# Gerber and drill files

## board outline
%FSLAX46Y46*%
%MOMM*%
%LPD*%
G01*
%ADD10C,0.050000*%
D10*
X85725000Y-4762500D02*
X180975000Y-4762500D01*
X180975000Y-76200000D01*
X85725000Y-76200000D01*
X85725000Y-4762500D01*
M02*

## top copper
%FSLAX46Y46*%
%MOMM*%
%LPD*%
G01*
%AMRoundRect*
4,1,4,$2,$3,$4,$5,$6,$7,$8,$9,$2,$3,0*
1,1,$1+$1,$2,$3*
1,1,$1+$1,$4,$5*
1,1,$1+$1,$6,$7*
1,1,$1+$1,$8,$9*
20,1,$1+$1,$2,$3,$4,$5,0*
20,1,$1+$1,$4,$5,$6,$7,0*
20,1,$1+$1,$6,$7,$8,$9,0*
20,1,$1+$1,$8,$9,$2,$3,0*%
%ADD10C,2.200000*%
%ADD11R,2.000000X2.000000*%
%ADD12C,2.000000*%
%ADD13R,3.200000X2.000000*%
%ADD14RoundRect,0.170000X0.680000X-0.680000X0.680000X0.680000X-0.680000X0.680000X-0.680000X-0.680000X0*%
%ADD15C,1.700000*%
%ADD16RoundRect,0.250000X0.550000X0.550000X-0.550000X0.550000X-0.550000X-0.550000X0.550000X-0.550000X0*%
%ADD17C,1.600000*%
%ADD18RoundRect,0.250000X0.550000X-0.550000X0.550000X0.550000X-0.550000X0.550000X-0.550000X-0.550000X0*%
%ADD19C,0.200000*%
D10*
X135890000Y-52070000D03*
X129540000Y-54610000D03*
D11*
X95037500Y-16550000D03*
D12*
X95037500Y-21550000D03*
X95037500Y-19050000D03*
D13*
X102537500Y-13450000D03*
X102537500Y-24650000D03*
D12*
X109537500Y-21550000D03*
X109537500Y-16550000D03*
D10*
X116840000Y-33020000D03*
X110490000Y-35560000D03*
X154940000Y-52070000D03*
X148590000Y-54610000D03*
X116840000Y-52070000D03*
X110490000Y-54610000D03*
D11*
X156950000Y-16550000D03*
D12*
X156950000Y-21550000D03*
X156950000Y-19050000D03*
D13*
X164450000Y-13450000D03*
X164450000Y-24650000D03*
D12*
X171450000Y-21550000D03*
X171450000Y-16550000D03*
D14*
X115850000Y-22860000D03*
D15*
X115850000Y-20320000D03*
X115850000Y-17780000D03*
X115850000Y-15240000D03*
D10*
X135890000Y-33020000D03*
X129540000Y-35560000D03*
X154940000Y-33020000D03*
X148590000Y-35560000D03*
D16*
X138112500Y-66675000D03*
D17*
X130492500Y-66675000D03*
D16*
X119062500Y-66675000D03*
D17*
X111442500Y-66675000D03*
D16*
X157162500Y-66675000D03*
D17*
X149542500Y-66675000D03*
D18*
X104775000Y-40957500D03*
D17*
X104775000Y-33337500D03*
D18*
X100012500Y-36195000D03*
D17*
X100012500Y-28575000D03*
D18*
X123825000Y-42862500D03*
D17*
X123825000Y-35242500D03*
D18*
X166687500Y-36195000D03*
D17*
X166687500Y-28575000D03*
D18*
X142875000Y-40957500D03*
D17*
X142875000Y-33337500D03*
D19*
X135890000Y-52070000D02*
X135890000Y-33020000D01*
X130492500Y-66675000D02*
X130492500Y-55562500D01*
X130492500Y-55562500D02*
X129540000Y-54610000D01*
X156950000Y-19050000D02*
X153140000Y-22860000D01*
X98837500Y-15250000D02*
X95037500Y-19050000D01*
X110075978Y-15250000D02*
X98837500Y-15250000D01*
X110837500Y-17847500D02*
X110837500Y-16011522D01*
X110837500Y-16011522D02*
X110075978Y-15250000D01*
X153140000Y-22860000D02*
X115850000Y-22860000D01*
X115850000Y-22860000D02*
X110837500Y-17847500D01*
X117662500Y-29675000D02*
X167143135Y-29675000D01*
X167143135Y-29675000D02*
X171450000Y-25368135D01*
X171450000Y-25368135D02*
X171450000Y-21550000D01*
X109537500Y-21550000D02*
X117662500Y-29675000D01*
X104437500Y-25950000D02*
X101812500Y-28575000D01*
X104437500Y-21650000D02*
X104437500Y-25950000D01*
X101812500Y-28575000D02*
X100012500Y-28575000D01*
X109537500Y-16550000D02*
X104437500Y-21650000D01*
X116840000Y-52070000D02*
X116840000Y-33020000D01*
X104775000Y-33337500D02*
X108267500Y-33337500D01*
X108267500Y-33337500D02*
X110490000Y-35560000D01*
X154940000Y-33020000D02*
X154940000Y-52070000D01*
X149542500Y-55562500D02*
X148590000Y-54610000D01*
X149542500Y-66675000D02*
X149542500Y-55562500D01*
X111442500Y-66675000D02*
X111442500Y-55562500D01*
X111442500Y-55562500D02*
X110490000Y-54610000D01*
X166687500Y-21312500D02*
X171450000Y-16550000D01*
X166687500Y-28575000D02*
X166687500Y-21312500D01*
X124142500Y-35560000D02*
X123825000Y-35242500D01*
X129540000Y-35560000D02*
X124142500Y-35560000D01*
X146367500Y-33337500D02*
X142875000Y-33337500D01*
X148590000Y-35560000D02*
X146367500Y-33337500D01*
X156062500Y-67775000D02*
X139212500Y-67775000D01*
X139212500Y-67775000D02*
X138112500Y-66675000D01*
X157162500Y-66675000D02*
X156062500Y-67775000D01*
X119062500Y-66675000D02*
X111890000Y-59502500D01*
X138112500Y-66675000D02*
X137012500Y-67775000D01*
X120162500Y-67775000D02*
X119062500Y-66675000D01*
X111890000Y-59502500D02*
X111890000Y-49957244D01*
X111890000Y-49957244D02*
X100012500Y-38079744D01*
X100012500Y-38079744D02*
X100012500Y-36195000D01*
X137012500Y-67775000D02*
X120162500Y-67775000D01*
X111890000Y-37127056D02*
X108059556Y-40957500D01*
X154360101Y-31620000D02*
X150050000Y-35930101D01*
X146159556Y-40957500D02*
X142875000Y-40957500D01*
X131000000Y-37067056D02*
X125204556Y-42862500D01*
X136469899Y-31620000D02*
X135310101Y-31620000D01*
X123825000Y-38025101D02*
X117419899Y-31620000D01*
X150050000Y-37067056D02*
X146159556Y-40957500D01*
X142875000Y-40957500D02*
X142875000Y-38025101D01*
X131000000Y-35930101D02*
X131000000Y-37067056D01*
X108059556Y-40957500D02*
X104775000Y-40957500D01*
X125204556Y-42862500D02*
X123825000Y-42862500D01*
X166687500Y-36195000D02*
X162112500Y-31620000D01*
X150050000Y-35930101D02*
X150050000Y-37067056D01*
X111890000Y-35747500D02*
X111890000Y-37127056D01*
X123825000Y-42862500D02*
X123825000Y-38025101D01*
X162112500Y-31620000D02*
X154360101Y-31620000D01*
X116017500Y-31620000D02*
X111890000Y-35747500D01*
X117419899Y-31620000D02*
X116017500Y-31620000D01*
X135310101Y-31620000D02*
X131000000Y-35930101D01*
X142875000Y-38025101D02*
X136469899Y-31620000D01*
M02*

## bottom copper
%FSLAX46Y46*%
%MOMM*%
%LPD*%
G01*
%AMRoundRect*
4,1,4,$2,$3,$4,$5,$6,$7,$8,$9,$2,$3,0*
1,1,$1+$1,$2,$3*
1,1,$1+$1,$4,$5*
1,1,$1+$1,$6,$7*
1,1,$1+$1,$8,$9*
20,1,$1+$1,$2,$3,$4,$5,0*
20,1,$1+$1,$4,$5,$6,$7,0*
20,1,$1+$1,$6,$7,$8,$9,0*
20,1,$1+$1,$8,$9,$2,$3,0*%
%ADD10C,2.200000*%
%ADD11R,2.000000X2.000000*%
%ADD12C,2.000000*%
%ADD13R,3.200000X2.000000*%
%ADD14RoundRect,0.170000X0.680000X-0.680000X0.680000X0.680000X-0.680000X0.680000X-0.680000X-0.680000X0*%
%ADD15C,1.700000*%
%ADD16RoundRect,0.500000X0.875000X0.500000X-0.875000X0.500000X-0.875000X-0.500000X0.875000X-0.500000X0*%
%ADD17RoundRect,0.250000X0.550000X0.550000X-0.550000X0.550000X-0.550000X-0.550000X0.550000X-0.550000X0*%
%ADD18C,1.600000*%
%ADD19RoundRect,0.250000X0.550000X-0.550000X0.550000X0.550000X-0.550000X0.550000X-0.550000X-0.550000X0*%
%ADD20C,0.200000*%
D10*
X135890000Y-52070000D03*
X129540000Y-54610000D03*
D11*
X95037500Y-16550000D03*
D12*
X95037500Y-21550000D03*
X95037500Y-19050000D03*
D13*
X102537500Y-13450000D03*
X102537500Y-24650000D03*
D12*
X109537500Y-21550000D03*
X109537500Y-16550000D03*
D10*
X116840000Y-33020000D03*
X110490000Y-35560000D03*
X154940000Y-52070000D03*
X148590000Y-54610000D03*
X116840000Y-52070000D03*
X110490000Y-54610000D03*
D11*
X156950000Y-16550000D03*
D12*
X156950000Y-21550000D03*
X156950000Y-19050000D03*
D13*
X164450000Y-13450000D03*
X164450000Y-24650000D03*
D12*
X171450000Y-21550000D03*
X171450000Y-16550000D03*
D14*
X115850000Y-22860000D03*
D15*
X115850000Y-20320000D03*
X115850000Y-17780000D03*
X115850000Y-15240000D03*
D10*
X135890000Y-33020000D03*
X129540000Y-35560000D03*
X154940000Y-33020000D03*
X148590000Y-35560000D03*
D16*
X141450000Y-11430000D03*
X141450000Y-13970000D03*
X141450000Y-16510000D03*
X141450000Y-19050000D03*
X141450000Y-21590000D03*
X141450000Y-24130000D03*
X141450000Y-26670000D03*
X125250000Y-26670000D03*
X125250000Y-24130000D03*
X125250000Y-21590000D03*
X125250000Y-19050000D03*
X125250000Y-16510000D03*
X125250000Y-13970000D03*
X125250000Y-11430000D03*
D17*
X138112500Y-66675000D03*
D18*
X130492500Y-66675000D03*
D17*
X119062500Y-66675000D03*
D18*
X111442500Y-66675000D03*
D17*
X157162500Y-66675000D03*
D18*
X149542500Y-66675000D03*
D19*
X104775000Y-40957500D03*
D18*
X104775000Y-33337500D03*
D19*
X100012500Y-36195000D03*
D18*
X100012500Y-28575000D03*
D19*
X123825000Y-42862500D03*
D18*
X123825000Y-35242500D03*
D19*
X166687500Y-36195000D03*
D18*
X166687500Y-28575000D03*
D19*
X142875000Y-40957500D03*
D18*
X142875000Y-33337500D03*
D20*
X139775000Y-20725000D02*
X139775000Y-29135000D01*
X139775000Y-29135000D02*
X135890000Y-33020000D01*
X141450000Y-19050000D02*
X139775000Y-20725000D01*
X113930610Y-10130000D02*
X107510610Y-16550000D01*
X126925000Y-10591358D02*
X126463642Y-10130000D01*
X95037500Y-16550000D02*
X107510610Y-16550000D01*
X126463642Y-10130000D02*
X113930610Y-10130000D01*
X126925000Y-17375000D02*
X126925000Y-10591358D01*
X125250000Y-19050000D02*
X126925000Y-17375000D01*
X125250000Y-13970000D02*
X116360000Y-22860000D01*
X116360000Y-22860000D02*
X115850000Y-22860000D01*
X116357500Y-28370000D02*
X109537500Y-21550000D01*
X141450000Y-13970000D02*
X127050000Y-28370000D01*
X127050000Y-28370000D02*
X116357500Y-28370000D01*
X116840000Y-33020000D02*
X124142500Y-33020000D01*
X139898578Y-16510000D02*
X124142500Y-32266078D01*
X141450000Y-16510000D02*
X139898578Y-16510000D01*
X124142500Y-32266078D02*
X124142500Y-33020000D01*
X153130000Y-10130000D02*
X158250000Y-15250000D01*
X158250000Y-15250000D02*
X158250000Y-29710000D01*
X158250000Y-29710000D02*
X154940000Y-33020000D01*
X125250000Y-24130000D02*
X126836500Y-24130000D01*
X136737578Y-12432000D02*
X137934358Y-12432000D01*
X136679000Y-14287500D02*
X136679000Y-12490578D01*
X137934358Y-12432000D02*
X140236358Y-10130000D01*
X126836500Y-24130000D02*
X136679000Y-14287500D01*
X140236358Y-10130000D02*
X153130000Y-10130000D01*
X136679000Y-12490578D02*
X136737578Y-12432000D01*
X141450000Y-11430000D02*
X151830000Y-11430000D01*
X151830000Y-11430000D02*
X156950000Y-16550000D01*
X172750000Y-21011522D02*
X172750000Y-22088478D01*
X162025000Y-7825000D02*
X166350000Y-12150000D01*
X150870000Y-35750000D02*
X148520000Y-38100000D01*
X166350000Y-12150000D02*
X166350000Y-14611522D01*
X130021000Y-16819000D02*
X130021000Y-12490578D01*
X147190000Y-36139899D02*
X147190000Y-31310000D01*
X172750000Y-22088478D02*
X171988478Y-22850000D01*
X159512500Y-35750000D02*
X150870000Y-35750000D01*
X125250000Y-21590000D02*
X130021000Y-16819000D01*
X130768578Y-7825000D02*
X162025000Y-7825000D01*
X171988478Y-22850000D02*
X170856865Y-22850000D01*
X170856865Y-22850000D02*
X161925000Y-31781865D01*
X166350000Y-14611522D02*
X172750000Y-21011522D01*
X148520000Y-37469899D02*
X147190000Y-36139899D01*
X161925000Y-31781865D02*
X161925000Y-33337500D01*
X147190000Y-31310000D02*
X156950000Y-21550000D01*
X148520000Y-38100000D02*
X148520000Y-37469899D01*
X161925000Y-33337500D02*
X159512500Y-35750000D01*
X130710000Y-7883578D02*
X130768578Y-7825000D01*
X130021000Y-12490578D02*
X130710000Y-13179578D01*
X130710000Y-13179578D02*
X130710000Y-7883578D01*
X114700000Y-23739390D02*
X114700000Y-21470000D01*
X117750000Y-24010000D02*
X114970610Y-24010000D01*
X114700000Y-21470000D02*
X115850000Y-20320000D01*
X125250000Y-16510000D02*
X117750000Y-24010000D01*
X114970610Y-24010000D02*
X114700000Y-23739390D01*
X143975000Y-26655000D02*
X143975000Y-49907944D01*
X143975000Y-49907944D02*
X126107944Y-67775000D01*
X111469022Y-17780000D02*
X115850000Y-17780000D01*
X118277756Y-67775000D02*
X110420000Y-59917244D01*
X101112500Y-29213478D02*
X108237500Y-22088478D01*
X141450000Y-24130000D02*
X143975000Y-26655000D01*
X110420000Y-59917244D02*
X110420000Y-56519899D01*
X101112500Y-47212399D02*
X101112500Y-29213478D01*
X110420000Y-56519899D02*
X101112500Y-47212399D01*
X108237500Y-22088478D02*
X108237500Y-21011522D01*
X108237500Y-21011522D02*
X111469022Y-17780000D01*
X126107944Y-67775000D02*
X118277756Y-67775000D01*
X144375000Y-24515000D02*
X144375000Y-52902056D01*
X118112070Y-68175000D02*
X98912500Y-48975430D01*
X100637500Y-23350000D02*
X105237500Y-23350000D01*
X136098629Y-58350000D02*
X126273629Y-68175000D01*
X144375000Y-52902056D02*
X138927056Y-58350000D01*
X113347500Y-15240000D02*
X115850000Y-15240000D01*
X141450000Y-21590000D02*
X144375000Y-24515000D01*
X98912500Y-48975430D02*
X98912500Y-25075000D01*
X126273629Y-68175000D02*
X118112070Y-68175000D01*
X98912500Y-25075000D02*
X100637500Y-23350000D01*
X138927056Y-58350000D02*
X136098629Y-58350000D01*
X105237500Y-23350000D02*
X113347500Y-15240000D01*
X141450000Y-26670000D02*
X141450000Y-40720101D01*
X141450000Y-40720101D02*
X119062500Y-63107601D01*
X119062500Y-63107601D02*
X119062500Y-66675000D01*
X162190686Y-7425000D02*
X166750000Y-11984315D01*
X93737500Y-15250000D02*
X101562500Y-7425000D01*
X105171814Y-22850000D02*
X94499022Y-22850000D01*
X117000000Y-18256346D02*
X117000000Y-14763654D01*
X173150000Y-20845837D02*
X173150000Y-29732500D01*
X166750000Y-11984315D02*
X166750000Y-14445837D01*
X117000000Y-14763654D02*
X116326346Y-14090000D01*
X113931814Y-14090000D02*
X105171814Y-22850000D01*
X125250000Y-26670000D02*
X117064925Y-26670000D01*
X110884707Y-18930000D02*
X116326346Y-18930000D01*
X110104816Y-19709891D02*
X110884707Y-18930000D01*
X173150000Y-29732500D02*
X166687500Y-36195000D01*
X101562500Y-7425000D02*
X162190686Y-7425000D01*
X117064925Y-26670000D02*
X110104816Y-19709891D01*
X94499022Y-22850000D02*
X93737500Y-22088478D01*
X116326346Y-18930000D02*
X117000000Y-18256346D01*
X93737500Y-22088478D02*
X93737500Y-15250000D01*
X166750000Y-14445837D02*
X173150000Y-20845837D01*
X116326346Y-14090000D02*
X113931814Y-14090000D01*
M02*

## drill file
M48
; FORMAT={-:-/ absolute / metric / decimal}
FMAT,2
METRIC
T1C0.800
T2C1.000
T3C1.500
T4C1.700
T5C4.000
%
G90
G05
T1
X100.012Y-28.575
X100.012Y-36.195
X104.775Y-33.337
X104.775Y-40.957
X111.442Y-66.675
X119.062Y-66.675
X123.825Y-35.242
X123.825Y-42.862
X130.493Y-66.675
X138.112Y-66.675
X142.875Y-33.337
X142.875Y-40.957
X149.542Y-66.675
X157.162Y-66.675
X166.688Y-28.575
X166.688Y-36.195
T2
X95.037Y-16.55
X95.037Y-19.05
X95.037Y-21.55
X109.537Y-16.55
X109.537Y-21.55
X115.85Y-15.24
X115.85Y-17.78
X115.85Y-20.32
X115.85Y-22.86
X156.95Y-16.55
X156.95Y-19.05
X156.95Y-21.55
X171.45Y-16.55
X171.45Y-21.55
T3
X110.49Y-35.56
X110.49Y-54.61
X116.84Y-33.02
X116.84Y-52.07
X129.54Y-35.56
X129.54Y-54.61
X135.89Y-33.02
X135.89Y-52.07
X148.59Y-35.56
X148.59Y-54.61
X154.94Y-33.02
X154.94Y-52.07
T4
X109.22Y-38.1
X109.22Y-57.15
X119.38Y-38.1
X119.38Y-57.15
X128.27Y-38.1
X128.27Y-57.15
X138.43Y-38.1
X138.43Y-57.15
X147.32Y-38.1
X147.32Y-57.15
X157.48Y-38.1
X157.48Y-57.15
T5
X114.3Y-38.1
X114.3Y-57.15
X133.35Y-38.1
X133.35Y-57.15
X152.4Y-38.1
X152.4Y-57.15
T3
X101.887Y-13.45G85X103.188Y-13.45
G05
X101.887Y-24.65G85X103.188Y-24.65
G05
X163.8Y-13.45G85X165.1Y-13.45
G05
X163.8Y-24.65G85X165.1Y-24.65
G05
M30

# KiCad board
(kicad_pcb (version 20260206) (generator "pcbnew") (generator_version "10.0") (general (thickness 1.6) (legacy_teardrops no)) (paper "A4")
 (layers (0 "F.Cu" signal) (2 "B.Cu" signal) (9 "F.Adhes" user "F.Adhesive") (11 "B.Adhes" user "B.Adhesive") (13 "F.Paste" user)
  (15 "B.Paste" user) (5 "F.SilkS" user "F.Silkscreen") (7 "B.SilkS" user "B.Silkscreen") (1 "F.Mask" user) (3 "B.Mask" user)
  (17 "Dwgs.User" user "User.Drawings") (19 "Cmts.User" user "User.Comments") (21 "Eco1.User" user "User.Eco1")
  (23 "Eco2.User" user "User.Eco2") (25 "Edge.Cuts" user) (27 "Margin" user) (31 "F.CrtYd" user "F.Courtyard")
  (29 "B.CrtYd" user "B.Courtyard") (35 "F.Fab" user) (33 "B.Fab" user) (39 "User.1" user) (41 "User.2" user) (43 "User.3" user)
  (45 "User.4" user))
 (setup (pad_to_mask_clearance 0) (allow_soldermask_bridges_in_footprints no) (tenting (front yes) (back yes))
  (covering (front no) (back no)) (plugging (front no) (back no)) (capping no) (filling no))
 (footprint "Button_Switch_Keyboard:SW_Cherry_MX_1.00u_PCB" (layer "F.Cu") (at 135.89 52.07)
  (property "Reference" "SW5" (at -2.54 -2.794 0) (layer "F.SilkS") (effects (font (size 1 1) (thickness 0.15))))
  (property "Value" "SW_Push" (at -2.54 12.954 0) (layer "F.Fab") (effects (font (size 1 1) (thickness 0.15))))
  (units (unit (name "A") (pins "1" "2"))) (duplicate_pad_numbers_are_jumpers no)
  (pad "" np_thru_hole circle (at -7.62 5.08) (size 1.7 1.7) (drill 1.7) (layers "*.Cu" "*.Mask"))
  (pad "" np_thru_hole circle (at -2.54 5.08) (size 4 4) (drill 4) (layers "*.Cu" "*.Mask"))
  (pad "" np_thru_hole circle (at 2.54 5.08) (size 1.7 1.7) (drill 1.7) (layers "*.Cu" "*.Mask"))
  (pad "1" thru_hole circle (at 0 0) (size 2.2 2.2) (drill 1.5) (layers "*.Cu" "*.Mask") (remove_unused_layers no) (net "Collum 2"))
  (pad "2" thru_hole circle (at -6.35 2.54) (size 2.2 2.2) (drill 1.5) (layers "*.Cu" "*.Mask") (remove_unused_layers no) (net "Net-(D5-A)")))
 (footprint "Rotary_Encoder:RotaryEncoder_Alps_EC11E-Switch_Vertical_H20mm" (layer "F.Cu") (at 95.0375 16.55)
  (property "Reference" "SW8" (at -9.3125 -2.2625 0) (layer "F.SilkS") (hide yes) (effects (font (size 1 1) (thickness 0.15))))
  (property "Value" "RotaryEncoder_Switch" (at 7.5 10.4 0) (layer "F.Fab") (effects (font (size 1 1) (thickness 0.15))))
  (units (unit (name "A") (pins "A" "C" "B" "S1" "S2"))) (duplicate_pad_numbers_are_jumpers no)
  (pad "A" thru_hole rect (at 0 0) (size 2 2) (drill 1) (layers "*.Cu" "*.Mask") (remove_unused_layers no) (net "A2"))
  (pad "B" thru_hole circle (at 0 5) (size 2 2) (drill 1) (layers "*.Cu" "*.Mask") (remove_unused_layers no) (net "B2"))
  (pad "C" thru_hole circle (at 0 2.5) (size 2 2) (drill 1) (layers "*.Cu" "*.Mask") (remove_unused_layers no) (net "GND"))
  (pad "MP" thru_hole rect (at 7.5 -3.1) (size 3.2 2) (drill oval 2.8 1.5) (layers "*.Cu" "*.Mask") (remove_unused_layers no))
  (pad "MP" thru_hole rect (at 7.5 8.1) (size 3.2 2) (drill oval 2.8 1.5) (layers "*.Cu" "*.Mask") (remove_unused_layers no))
  (pad "S1" thru_hole circle (at 14.5 5) (size 2 2) (drill 1) (layers "*.Cu" "*.Mask") (remove_unused_layers no) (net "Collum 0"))
  (pad "S2" thru_hole circle (at 14.5 0) (size 2 2) (drill 1) (layers "*.Cu" "*.Mask") (remove_unused_layers no) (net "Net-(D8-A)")))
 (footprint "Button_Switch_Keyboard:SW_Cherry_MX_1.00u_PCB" (layer "F.Cu") (at 116.84 33.02)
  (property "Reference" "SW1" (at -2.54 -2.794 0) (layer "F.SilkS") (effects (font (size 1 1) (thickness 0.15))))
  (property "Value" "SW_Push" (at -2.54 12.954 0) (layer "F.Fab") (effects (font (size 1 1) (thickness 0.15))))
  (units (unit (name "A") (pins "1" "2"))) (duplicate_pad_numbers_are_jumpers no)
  (pad "" np_thru_hole circle (at -7.62 5.08) (size 1.7 1.7) (drill 1.7) (layers "*.Cu" "*.Mask"))
  (pad "" np_thru_hole circle (at -2.54 5.08) (size 4 4) (drill 4) (layers "*.Cu" "*.Mask"))
  (pad "" np_thru_hole circle (at 2.54 5.08) (size 1.7 1.7) (drill 1.7) (layers "*.Cu" "*.Mask"))
  (pad "1" thru_hole circle (at 0 0) (size 2.2 2.2) (drill 1.5) (layers "*.Cu" "*.Mask") (remove_unused_layers no) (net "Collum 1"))
  (pad "2" thru_hole circle (at -6.35 2.54) (size 2.2 2.2) (drill 1.5) (layers "*.Cu" "*.Mask") (remove_unused_layers no) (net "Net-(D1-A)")))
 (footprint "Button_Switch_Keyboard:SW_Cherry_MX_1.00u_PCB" (layer "F.Cu") (at 154.94 52.07)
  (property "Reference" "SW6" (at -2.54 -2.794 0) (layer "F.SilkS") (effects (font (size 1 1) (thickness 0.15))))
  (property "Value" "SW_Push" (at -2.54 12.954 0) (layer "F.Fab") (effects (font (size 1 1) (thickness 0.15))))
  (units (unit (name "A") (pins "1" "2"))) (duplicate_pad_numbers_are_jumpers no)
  (pad "" np_thru_hole circle (at -7.62 5.08) (size 1.7 1.7) (drill 1.7) (layers "*.Cu" "*.Mask"))
  (pad "" np_thru_hole circle (at -2.54 5.08) (size 4 4) (drill 4) (layers "*.Cu" "*.Mask"))
  (pad "" np_thru_hole circle (at 2.54 5.08) (size 1.7 1.7) (drill 1.7) (layers "*.Cu" "*.Mask"))
  (pad "1" thru_hole circle (at 0 0) (size 2.2 2.2) (drill 1.5) (layers "*.Cu" "*.Mask") (remove_unused_layers no) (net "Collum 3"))
  (pad "2" thru_hole circle (at -6.35 2.54) (size 2.2 2.2) (drill 1.5) (layers "*.Cu" "*.Mask") (remove_unused_layers no) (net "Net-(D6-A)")))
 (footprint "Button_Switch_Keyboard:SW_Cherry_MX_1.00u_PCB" (layer "F.Cu") (at 116.84 52.07)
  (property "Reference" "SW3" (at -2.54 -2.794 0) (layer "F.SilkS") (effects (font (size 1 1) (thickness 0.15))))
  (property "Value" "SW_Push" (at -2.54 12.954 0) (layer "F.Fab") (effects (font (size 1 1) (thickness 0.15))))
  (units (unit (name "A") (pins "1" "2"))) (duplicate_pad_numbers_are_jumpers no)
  (pad "" np_thru_hole circle (at -7.62 5.08) (size 1.7 1.7) (drill 1.7) (layers "*.Cu" "*.Mask"))
  (pad "" np_thru_hole circle (at -2.54 5.08) (size 4 4) (drill 4) (layers "*.Cu" "*.Mask"))
  (pad "" np_thru_hole circle (at 2.54 5.08) (size 1.7 1.7) (drill 1.7) (layers "*.Cu" "*.Mask"))
  (pad "1" thru_hole circle (at 0 0) (size 2.2 2.2) (drill 1.5) (layers "*.Cu" "*.Mask") (remove_unused_layers no) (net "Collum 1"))
  (pad "2" thru_hole circle (at -6.35 2.54) (size 2.2 2.2) (drill 1.5) (layers "*.Cu" "*.Mask") (remove_unused_layers no) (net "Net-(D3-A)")))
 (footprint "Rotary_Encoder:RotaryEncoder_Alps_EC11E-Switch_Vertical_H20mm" (layer "F.Cu") (at 156.95 16.55)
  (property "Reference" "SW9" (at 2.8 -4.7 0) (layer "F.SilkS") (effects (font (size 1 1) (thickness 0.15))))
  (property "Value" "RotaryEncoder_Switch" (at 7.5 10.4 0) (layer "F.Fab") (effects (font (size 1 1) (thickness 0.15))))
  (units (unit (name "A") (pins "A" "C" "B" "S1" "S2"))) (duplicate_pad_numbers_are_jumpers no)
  (pad "A" thru_hole rect (at 0 0) (size 2 2) (drill 1) (layers "*.Cu" "*.Mask") (remove_unused_layers no) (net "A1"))
  (pad "B" thru_hole circle (at 0 5) (size 2 2) (drill 1) (layers "*.Cu" "*.Mask") (remove_unused_layers no) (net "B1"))
  (pad "C" thru_hole circle (at 0 2.5) (size 2 2) (drill 1) (layers "*.Cu" "*.Mask") (remove_unused_layers no) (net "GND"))
  (pad "MP" thru_hole rect (at 7.5 -3.1) (size 3.2 2) (drill oval 2.8 1.5) (layers "*.Cu" "*.Mask") (remove_unused_layers no))
  (pad "MP" thru_hole rect (at 7.5 8.1) (size 3.2 2) (drill oval 2.8 1.5) (layers "*.Cu" "*.Mask") (remove_unused_layers no))
  (pad "S1" thru_hole circle (at 14.5 5) (size 2 2) (drill 1) (layers "*.Cu" "*.Mask") (remove_unused_layers no) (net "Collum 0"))
  (pad "S2" thru_hole circle (at 14.5 0) (size 2 2) (drill 1) (layers "*.Cu" "*.Mask") (remove_unused_layers no) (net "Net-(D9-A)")))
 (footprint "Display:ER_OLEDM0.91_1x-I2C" (layer "F.Cu") (at 115.85 22.86 90)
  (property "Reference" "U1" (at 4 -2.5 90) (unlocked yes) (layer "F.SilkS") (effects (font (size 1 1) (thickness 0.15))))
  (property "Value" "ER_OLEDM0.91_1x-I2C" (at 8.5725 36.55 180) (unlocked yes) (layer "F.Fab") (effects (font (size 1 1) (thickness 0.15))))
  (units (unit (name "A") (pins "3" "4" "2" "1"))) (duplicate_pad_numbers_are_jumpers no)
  (pad "1" thru_hole roundrect (at 0 0 90) (size 1.7 1.7) (drill 1) (layers "*.Cu" "*.Mask") (remove_unused_layers no)
   (roundrect_rratio 0.1) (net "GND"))
  (pad "2" thru_hole circle (at 2.54 0 90) (size 1.7 1.7) (drill 1) (layers "*.Cu" "*.Mask") (remove_unused_layers no) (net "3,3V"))
  (pad "3" thru_hole circle (at 5.08 0 90) (size 1.7 1.7) (drill 1) (layers "*.Cu" "*.Mask") (remove_unused_layers no) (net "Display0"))
  (pad "4" thru_hole circle (at 7.62 0 90) (size 1.7 1.7) (drill 1) (layers "*.Cu" "*.Mask") (remove_unused_layers no) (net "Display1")))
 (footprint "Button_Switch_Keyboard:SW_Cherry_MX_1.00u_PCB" (layer "F.Cu") (at 135.89 33.02)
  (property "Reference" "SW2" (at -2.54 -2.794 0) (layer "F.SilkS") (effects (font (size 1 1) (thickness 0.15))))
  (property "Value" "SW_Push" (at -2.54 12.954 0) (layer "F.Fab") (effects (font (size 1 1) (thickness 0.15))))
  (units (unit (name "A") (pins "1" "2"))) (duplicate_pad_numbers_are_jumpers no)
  (pad "" np_thru_hole circle (at -7.62 5.08) (size 1.7 1.7) (drill 1.7) (layers "*.Cu" "*.Mask"))
  (pad "" np_thru_hole circle (at -2.54 5.08) (size 4 4) (drill 4) (layers "*.Cu" "*.Mask"))
  (pad "" np_thru_hole circle (at 2.54 5.08) (size 1.7 1.7) (drill 1.7) (layers "*.Cu" "*.Mask"))
  (pad "1" thru_hole circle (at 0 0) (size 2.2 2.2) (drill 1.5) (layers "*.Cu" "*.Mask") (remove_unused_layers no) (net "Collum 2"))
  (pad "2" thru_hole circle (at -6.35 2.54) (size 2.2 2.2) (drill 1.5) (layers "*.Cu" "*.Mask") (remove_unused_layers no) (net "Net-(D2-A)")))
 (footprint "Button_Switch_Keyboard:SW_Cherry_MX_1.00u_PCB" (layer "F.Cu") (at 154.94 33.02)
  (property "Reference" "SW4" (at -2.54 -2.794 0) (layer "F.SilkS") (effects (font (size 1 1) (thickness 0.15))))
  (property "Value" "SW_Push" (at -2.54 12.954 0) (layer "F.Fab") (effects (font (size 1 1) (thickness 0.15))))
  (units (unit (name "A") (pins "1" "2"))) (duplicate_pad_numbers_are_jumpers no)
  (pad "" np_thru_hole circle (at -7.62 5.08) (size 1.7 1.7) (drill 1.7) (layers "*.Cu" "*.Mask"))
  (pad "" np_thru_hole circle (at -2.54 5.08) (size 4 4) (drill 4) (layers "*.Cu" "*.Mask"))
  (pad "" np_thru_hole circle (at 2.54 5.08) (size 1.7 1.7) (drill 1.7) (layers "*.Cu" "*.Mask"))
  (pad "1" thru_hole circle (at 0 0) (size 2.2 2.2) (drill 1.5) (layers "*.Cu" "*.Mask") (remove_unused_layers no) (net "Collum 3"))
  (pad "2" thru_hole circle (at -6.35 2.54) (size 2.2 2.2) (drill 1.5) (layers "*.Cu" "*.Mask") (remove_unused_layers no) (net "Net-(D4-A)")))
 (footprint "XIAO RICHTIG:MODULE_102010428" (layer "B.Cu") (at 133.35 19.05 180)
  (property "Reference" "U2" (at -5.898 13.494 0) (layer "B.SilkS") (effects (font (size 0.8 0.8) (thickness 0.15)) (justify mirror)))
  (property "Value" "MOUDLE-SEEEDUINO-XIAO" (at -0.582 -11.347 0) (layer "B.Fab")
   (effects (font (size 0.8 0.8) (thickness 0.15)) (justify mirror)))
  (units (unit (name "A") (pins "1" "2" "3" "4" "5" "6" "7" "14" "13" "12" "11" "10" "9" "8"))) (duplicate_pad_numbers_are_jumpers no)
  (pad "1" smd roundrect (at -8.1 7.62 180) (size 2.75 2) (layers "B.Cu" "B.Mask" "B.Paste") (roundrect_rratio 0.25) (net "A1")
   (solder_mask_margin 0.102))
  (pad "2" smd roundrect (at -8.1 5.08 180) (size 2.75 2) (layers "B.Cu" "B.Mask" "B.Paste") (roundrect_rratio 0.25) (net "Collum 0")
   (solder_mask_margin 0.102))
  (pad "3" smd roundrect (at -8.1 2.54 180) (size 2.75 2) (layers "B.Cu" "B.Mask" "B.Paste") (roundrect_rratio 0.25) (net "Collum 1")
   (solder_mask_margin 0.102))
  (pad "4" smd roundrect (at -8.1 0 180) (size 2.75 2) (layers "B.Cu" "B.Mask" "B.Paste") (roundrect_rratio 0.25) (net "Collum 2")
   (solder_mask_margin 0.102))
  (pad "5" smd roundrect (at -8.1 -2.54 180) (size 2.75 2) (layers "B.Cu" "B.Mask" "B.Paste") (roundrect_rratio 0.25) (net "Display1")
   (solder_mask_margin 0.102))
  (pad "6" smd roundrect (at -8.1 -5.08 180) (size 2.75 2) (layers "B.Cu" "B.Mask" "B.Paste") (roundrect_rratio 0.25) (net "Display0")
   (solder_mask_margin 0.102))
  (pad "7" smd roundrect (at -8.1 -7.62 180) (size 2.75 2) (layers "B.Cu" "B.Mask" "B.Paste") (roundrect_rratio 0.25) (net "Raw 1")
   (solder_mask_margin 0.102))
  (pad "8" smd roundrect (at 8.1 -7.62 180) (size 2.75 2) (layers "B.Cu" "B.Mask" "B.Paste") (roundrect_rratio 0.25) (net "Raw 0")
   (solder_mask_margin 0.102))
  (pad "9" smd roundrect (at 8.1 -5.08 180) (size 2.75 2) (layers "B.Cu" "B.Mask" "B.Paste") (roundrect_rratio 0.25) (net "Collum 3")
   (solder_mask_margin 0.102))
  (pad "10" smd roundrect (at 8.1 -2.54 180) (size 2.75 2) (layers "B.Cu" "B.Mask" "B.Paste") (roundrect_rratio 0.25) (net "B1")
   (solder_mask_margin 0.102))
  (pad "11" smd roundrect (at 8.1 0 180) (size 2.75 2) (layers "B.Cu" "B.Mask" "B.Paste") (roundrect_rratio 0.25) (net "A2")
   (solder_mask_margin 0.102))
  (pad "12" smd roundrect (at 8.1 2.54 180) (size 2.75 2) (layers "B.Cu" "B.Mask" "B.Paste") (roundrect_rratio 0.25) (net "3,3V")
   (solder_mask_margin 0.102))
  (pad "13" smd roundrect (at 8.1 5.08 180) (size 2.75 2) (layers "B.Cu" "B.Mask" "B.Paste") (roundrect_rratio 0.25) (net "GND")
   (solder_mask_margin 0.102))
  (pad "14" smd roundrect (at 8.1 7.62 180) (size 2.75 2) (layers "B.Cu" "B.Mask" "B.Paste") (roundrect_rratio 0.25)
   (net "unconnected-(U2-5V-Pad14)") (solder_mask_margin 0.102))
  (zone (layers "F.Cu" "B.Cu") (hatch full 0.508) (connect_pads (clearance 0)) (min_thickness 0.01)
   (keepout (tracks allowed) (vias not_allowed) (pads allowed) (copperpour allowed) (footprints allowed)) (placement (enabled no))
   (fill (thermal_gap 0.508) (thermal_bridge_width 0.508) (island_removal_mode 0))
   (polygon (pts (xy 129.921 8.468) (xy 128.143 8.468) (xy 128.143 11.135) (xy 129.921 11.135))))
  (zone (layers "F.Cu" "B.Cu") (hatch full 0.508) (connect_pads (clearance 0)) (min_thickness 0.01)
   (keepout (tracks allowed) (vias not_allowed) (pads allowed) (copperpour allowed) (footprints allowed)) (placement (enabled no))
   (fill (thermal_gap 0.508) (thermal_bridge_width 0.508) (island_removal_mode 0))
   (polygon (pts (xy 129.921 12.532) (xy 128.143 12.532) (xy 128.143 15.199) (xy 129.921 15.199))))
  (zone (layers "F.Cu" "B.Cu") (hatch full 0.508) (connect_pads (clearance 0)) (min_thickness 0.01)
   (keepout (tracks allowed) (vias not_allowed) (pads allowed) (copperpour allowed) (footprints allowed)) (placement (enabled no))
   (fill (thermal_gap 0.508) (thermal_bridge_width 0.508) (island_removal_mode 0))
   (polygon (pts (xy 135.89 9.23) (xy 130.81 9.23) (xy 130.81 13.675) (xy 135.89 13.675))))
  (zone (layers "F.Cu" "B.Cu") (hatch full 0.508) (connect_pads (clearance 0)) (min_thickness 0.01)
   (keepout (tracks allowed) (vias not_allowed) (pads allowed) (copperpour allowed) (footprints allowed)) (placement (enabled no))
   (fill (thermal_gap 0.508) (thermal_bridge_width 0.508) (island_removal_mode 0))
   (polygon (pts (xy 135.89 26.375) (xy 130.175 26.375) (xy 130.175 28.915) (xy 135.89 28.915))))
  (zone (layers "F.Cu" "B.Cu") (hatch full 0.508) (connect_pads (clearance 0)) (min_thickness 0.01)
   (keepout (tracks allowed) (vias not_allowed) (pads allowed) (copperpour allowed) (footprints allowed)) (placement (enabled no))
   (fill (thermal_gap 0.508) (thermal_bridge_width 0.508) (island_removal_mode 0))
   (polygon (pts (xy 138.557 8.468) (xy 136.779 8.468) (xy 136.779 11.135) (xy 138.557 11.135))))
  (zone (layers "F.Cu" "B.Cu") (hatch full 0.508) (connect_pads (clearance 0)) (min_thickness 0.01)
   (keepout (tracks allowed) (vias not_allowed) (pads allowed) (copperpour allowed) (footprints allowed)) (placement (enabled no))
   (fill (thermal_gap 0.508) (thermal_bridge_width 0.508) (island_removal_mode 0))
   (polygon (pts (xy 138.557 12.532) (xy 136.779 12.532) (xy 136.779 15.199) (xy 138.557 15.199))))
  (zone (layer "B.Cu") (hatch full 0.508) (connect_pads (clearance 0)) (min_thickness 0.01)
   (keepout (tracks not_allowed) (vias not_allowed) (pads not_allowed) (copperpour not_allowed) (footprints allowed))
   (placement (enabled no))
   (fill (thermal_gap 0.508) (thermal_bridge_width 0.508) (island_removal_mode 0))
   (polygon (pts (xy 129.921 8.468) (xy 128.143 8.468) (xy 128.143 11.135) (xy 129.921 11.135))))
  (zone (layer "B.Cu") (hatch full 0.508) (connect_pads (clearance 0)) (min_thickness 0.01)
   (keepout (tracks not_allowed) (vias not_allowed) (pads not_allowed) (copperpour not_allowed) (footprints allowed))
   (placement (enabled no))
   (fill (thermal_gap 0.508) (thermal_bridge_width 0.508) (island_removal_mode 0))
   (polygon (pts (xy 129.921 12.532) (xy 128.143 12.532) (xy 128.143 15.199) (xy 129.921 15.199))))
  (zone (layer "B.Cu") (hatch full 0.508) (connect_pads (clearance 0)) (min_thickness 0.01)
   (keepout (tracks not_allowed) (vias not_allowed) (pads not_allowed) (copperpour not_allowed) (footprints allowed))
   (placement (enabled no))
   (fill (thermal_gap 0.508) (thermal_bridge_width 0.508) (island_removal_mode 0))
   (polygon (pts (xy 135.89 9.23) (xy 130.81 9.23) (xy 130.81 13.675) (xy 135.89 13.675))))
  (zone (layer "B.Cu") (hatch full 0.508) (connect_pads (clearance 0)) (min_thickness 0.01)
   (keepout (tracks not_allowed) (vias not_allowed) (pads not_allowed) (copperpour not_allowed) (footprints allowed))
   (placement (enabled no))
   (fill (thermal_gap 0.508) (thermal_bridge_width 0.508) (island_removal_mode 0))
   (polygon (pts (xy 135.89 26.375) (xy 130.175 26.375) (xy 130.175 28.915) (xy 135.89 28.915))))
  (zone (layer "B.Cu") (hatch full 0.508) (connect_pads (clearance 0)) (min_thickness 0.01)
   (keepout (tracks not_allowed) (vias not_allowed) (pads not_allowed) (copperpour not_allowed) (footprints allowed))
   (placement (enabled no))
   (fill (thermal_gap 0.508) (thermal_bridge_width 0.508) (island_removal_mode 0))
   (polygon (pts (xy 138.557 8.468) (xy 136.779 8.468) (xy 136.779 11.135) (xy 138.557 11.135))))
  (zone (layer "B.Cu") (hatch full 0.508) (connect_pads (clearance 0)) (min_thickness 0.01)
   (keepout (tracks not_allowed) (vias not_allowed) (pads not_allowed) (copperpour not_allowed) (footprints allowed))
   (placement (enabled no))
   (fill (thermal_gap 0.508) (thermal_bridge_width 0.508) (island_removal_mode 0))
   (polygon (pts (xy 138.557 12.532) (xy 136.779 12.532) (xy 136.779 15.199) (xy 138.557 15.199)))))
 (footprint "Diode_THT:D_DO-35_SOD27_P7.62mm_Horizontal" (layer "B.Cu") (at 138.1125 66.675 180)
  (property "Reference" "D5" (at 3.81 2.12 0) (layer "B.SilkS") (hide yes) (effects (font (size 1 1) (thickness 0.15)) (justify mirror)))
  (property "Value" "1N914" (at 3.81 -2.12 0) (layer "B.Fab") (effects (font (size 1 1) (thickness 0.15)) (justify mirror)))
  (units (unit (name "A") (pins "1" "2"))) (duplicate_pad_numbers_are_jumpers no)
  (pad "1" thru_hole roundrect (at 0 0 180) (size 1.6 1.6) (drill 0.8) (layers "*.Cu" "*.Mask") (remove_unused_layers no)
   (roundrect_rratio 0.15625) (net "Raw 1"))
  (pad "2" thru_hole circle (at 7.62 0 180) (size 1.6 1.6) (drill 0.8) (layers "*.Cu" "*.Mask") (remove_unused_layers no) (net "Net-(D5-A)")))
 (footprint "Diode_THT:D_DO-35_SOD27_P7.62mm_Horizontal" (layer "B.Cu") (at 119.0625 66.675 180)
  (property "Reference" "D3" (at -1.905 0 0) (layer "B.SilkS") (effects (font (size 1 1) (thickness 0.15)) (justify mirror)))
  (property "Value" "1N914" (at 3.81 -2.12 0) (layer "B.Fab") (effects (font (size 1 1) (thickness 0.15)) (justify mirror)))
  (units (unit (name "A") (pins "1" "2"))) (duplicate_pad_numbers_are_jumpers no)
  (pad "1" thru_hole roundrect (at 0 0 180) (size 1.6 1.6) (drill 0.8) (layers "*.Cu" "*.Mask") (remove_unused_layers no)
   (roundrect_rratio 0.15625) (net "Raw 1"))
  (pad "2" thru_hole circle (at 7.62 0 180) (size 1.6 1.6) (drill 0.8) (layers "*.Cu" "*.Mask") (remove_unused_layers no) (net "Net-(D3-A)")))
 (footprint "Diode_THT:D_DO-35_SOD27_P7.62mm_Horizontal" (layer "B.Cu") (at 157.1625 66.675 180)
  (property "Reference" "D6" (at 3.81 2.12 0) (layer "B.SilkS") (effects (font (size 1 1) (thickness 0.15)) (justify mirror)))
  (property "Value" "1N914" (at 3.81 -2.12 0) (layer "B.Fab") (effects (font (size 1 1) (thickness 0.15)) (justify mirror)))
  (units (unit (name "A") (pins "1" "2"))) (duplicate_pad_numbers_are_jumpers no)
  (pad "1" thru_hole roundrect (at 0 0 180) (size 1.6 1.6) (drill 0.8) (layers "*.Cu" "*.Mask") (remove_unused_layers no)
   (roundrect_rratio 0.15625) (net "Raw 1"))
  (pad "2" thru_hole circle (at 7.62 0 180) (size 1.6 1.6) (drill 0.8) (layers "*.Cu" "*.Mask") (remove_unused_layers no) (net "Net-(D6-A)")))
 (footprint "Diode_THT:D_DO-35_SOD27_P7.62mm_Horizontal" (layer "B.Cu") (at 104.775 40.9575 90)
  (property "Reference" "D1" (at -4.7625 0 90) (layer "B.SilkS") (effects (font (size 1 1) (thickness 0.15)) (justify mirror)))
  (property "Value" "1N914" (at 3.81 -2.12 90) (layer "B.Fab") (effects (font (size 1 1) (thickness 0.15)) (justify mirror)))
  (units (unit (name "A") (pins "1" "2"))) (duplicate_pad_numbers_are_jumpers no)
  (pad "1" thru_hole roundrect (at 0 0 90) (size 1.6 1.6) (drill 0.8) (layers "*.Cu" "*.Mask") (remove_unused_layers no)
   (roundrect_rratio 0.15625) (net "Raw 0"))
  (pad "2" thru_hole circle (at 7.62 0 90) (size 1.6 1.6) (drill 0.8) (layers "*.Cu" "*.Mask") (remove_unused_layers no) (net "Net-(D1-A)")))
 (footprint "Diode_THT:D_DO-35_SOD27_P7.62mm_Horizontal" (layer "B.Cu") (at 100.0125 36.195 90)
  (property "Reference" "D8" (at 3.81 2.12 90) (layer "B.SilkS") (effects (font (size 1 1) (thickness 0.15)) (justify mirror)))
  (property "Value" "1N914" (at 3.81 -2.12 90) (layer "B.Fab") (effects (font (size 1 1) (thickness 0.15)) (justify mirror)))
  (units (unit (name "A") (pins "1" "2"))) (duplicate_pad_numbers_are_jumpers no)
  (pad "1" thru_hole roundrect (at 0 0 90) (size 1.6 1.6) (drill 0.8) (layers "*.Cu" "*.Mask") (remove_unused_layers no)
   (roundrect_rratio 0.15625) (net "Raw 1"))
  (pad "2" thru_hole circle (at 7.62 0 90) (size 1.6 1.6) (drill 0.8) (layers "*.Cu" "*.Mask") (remove_unused_layers no) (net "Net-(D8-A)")))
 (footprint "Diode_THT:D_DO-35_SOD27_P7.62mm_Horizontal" (layer "B.Cu") (at 123.825 42.8625 90)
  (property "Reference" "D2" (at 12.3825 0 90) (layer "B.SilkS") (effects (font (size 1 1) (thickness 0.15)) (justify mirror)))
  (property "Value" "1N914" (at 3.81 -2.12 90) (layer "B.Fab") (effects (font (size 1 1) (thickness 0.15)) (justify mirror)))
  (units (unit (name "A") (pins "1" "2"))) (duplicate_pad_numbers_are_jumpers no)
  (pad "1" thru_hole roundrect (at 0 0 90) (size 1.6 1.6) (drill 0.8) (layers "*.Cu" "*.Mask") (remove_unused_layers no)
   (roundrect_rratio 0.15625) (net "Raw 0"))
  (pad "2" thru_hole circle (at 7.62 0 90) (size 1.6 1.6) (drill 0.8) (layers "*.Cu" "*.Mask") (remove_unused_layers no) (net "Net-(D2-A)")))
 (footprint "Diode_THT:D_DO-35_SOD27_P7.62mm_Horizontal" (layer "B.Cu") (at 166.6875 36.195 90)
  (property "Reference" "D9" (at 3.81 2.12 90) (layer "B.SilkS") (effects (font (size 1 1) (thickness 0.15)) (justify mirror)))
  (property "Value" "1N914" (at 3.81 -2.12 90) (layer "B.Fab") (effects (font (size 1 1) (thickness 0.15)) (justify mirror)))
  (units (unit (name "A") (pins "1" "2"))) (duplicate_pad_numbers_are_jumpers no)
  (pad "1" thru_hole roundrect (at 0 0 90) (size 1.6 1.6) (drill 0.8) (layers "*.Cu" "*.Mask") (remove_unused_layers no)
   (roundrect_rratio 0.15625) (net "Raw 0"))
  (pad "2" thru_hole circle (at 7.62 0 90) (size 1.6 1.6) (drill 0.8) (layers "*.Cu" "*.Mask") (remove_unused_layers no) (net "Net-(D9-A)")))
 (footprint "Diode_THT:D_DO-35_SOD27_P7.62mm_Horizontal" (layer "B.Cu") (at 142.875 40.9575 90)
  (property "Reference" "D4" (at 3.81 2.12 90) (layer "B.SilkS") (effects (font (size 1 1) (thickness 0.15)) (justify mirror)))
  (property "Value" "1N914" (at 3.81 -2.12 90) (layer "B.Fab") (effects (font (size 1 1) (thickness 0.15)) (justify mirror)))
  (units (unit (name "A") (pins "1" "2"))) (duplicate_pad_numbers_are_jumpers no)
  (pad "1" thru_hole roundrect (at 0 0 90) (size 1.6 1.6) (drill 0.8) (layers "*.Cu" "*.Mask") (remove_unused_layers no)
   (roundrect_rratio 0.15625) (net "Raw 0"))
  (pad "2" thru_hole circle (at 7.62 0 90) (size 1.6 1.6) (drill 0.8) (layers "*.Cu" "*.Mask") (remove_unused_layers no) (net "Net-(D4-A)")))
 (gr_rect (start 85.725 4.7625) (end 180.975 76.2) (stroke (width 0.05) (type default)) (fill no) (layer "Edge.Cuts"))
 (segment (start 135.89 52.07) (end 135.89 33.02) (width 0.2) (layer "F.Cu") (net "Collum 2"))
 (segment (start 139.775 20.725) (end 139.775 29.135) (width 0.2) (layer "B.Cu") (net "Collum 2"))
 (segment (start 139.775 29.135) (end 135.89 33.02) (width 0.2) (layer "B.Cu") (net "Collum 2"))
 (segment (start 141.45 19.05) (end 139.775 20.725) (width 0.2) (layer "B.Cu") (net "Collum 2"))
 (segment (start 130.4925 66.675) (end 130.4925 55.5625) (width 0.2) (layer "F.Cu") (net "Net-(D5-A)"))
 (segment (start 130.4925 55.5625) (end 129.54 54.61) (width 0.2) (layer "F.Cu") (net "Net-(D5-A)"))
 (segment (start 113.93061 10.13) (end 107.51061 16.55) (width 0.2) (layer "B.Cu") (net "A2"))
 (segment (start 126.925 10.591358) (end 126.463642 10.13) (width 0.2) (layer "B.Cu") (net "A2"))
 (segment (start 95.0375 16.55) (end 107.51061 16.55) (width 0.2) (layer "B.Cu") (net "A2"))
 (segment (start 126.463642 10.13) (end 113.93061 10.13) (width 0.2) (layer "B.Cu") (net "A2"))
 (segment (start 126.925 17.375) (end 126.925 10.591358) (width 0.2) (layer "B.Cu") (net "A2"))
 (segment (start 125.25 19.05) (end 126.925 17.375) (width 0.2) (layer "B.Cu") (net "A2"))
 (segment (start 156.95 19.05) (end 153.14 22.86) (width 0.2) (layer "F.Cu") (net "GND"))
 (segment (start 98.8375 15.25) (end 95.0375 19.05) (width 0.2) (layer "F.Cu") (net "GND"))
 (segment (start 110.075978 15.25) (end 98.8375 15.25) (width 0.2) (layer "F.Cu") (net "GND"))
 (segment (start 110.8375 17.8475) (end 110.8375 16.011522) (width 0.2) (layer "F.Cu") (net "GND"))
 (segment (start 110.8375 16.011522) (end 110.075978 15.25) (width 0.2) (layer "F.Cu") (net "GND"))
 (segment (start 153.14 22.86) (end 115.85 22.86) (width 0.2) (layer "F.Cu") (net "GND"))
 (segment (start 115.85 22.86) (end 110.8375 17.8475) (width 0.2) (layer "F.Cu") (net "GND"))
 (segment (start 125.25 13.97) (end 116.36 22.86) (width 0.2) (layer "B.Cu") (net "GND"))
 (segment (start 116.36 22.86) (end 115.85 22.86) (width 0.2) (layer "B.Cu") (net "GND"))
 (segment (start 117.6625 29.675) (end 167.143135 29.675) (width 0.2) (layer "F.Cu") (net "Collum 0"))
 (segment (start 167.143135 29.675) (end 171.45 25.368135) (width 0.2) (layer "F.Cu") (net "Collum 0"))
 (segment (start 171.45 25.368135) (end 171.45 21.55) (width 0.2) (layer "F.Cu") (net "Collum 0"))
 (segment (start 109.5375 21.55) (end 117.6625 29.675) (width 0.2) (layer "F.Cu") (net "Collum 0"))
 (segment (start 116.3575 28.37) (end 109.5375 21.55) (width 0.2) (layer "B.Cu") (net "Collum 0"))
 (segment (start 141.45 13.97) (end 127.05 28.37) (width 0.2) (layer "B.Cu") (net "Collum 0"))
 (segment (start 127.05 28.37) (end 116.3575 28.37) (width 0.2) (layer "B.Cu") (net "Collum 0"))
 (segment (start 104.4375 25.95) (end 101.8125 28.575) (width 0.2) (layer "F.Cu") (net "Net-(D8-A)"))
 (segment (start 104.4375 21.65) (end 104.4375 25.95) (width 0.2) (layer "F.Cu") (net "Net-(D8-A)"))
 (segment (start 101.8125 28.575) (end 100.0125 28.575) (width 0.2) (layer "F.Cu") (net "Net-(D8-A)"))
 (segment (start 109.5375 16.55) (end 104.4375 21.65) (width 0.2) (layer "F.Cu") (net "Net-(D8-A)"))
 (segment (start 116.84 52.07) (end 116.84 33.02) (width 0.2) (layer "F.Cu") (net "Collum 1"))
 (segment (start 116.84 33.02) (end 124.1425 33.02) (width 0.2) (layer "B.Cu") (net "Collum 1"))
 (segment (start 139.898578 16.51) (end 124.1425 32.266078) (width 0.2) (layer "B.Cu") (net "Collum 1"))
 (segment (start 141.45 16.51) (end 139.898578 16.51) (width 0.2) (layer "B.Cu") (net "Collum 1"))
 (segment (start 124.1425 32.266078) (end 124.1425 33.02) (width 0.2) (layer "B.Cu") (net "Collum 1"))
 (segment (start 104.775 33.3375) (end 108.2675 33.3375) (width 0.2) (layer "F.Cu") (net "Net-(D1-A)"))
 (segment (start 108.2675 33.3375) (end 110.49 35.56) (width 0.2) (layer "F.Cu") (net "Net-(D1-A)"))
 (segment (start 154.94 33.02) (end 154.94 52.07) (width 0.2) (layer "F.Cu") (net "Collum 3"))
 (segment (start 153.13 10.13) (end 158.25 15.25) (width 0.2) (layer "B.Cu") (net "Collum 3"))
 (segment (start 158.25 15.25) (end 158.25 29.71) (width 0.2) (layer "B.Cu") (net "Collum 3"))
 (segment (start 158.25 29.71) (end 154.94 33.02) (width 0.2) (layer "B.Cu") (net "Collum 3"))
 (segment (start 125.25 24.13) (end 126.8365 24.13) (width 0.2) (layer "B.Cu") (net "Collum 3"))
 (segment (start 136.737578 12.432) (end 137.934358 12.432) (width 0.2) (layer "B.Cu") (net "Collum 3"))
 (segment (start 136.679 14.2875) (end 136.679 12.490578) (width 0.2) (layer "B.Cu") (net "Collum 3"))
 (segment (start 137.934358 12.432) (end 140.236358 10.13) (width 0.2) (layer "B.Cu") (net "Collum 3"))
 (segment (start 126.8365 24.13) (end 136.679 14.2875) (width 0.2) (layer "B.Cu") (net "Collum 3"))
 (segment (start 140.236358 10.13) (end 153.13 10.13) (width 0.2) (layer "B.Cu") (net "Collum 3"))
 (segment (start 136.679 12.490578) (end 136.737578 12.432) (width 0.2) (layer "B.Cu") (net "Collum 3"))
 (segment (start 149.5425 55.5625) (end 148.59 54.61) (width 0.2) (layer "F.Cu") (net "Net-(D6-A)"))
 (segment (start 149.5425 66.675) (end 149.5425 55.5625) (width 0.2) (layer "F.Cu") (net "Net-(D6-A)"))
 (segment (start 111.4425 66.675) (end 111.4425 55.5625) (width 0.2) (layer "F.Cu") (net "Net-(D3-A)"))
 (segment (start 111.4425 55.5625) (end 110.49 54.61) (width 0.2) (layer "F.Cu") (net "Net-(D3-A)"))
 (segment (start 141.45 11.43) (end 151.83 11.43) (width 0.2) (layer "B.Cu") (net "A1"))
 (segment (start 151.83 11.43) (end 156.95 16.55) (width 0.2) (layer "B.Cu") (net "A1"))
 (segment (start 172.75 21.011522) (end 172.75 22.088478) (width 0.2) (layer "B.Cu") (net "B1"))
 (segment (start 162.025 7.825) (end 166.35 12.15) (width 0.2) (layer "B.Cu") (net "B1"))
 (segment (start 150.87 35.75) (end 148.52 38.1) (width 0.2) (layer "B.Cu") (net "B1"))
 (segment (start 166.35 12.15) (end 166.35 14.611522) (width 0.2) (layer "B.Cu") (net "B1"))
 (segment (start 130.021 16.819) (end 130.021 12.490578) (width 0.2) (layer "B.Cu") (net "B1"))
 (segment (start 147.19 36.139899) (end 147.19 31.31) (width 0.2) (layer "B.Cu") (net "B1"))
 (segment (start 172.75 22.088478) (end 171.988478 22.85) (width 0.2) (layer "B.Cu") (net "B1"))
 (segment (start 159.5125 35.75) (end 150.87 35.75) (width 0.2) (layer "B.Cu") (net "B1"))
 (segment (start 125.25 21.59) (end 130.021 16.819) (width 0.2) (layer "B.Cu") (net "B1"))
 (segment (start 130.768578 7.825) (end 162.025 7.825) (width 0.2) (layer "B.Cu") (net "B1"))
 (segment (start 171.988478 22.85) (end 170.856865 22.85) (width 0.2) (layer "B.Cu") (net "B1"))
 (segment (start 170.856865 22.85) (end 161.925 31.781865) (width 0.2) (layer "B.Cu") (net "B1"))
 (segment (start 166.35 14.611522) (end 172.75 21.011522) (width 0.2) (layer "B.Cu") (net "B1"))
 (segment (start 148.52 37.469899) (end 147.19 36.139899) (width 0.2) (layer "B.Cu") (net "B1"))
 (segment (start 161.925 31.781865) (end 161.925 33.3375) (width 0.2) (layer "B.Cu") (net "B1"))
 (segment (start 147.19 31.31) (end 156.95 21.55) (width 0.2) (layer "B.Cu") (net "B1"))
 (segment (start 148.52 38.1) (end 148.52 37.469899) (width 0.2) (layer "B.Cu") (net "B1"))
 (segment (start 161.925 33.3375) (end 159.5125 35.75) (width 0.2) (layer "B.Cu") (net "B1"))
 (segment (start 130.71 7.883578) (end 130.768578 7.825) (width 0.2) (layer "B.Cu") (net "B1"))
 (segment (start 130.021 12.490578) (end 130.71 13.179578) (width 0.2) (layer "B.Cu") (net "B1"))
 (segment (start 130.71 13.179578) (end 130.71 7.883578) (width 0.2) (layer "B.Cu") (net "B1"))
 (segment (start 166.6875 21.3125) (end 171.45 16.55) (width 0.2) (layer "F.Cu") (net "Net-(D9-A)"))
 (segment (start 166.6875 28.575) (end 166.6875 21.3125) (width 0.2) (layer "F.Cu") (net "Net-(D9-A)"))
 (segment (start 114.7 23.73939) (end 114.7 21.47) (width 0.2) (layer "B.Cu") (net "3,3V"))
 (segment (start 117.75 24.01) (end 114.97061 24.01) (width 0.2) (layer "B.Cu") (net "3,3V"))
 (segment (start 114.7 21.47) (end 115.85 20.32) (width 0.2) (layer "B.Cu") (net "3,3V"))
 (segment (start 125.25 16.51) (end 117.75 24.01) (width 0.2) (layer "B.Cu") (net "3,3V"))
 (segment (start 114.97061 24.01) (end 114.7 23.73939) (width 0.2) (layer "B.Cu") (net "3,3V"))
 (segment (start 143.975 26.655) (end 143.975 49.907944) (width 0.2) (layer "B.Cu") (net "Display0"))
 (segment (start 143.975 49.907944) (end 126.107944 67.775) (width 0.2) (layer "B.Cu") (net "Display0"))
 (segment (start 111.469022 17.78) (end 115.85 17.78) (width 0.2) (layer "B.Cu") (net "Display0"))
 (segment (start 118.277756 67.775) (end 110.42 59.917244) (width 0.2) (layer "B.Cu") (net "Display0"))
 (segment (start 101.1125 29.213478) (end 108.2375 22.088478) (width 0.2) (layer "B.Cu") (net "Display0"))
 (segment (start 141.45 24.13) (end 143.975 26.655) (width 0.2) (layer "B.Cu") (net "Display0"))
 (segment (start 110.42 59.917244) (end 110.42 56.519899) (width 0.2) (layer "B.Cu") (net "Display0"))
 (segment (start 101.1125 47.212399) (end 101.1125 29.213478) (width 0.2) (layer "B.Cu") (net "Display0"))
 (segment (start 110.42 56.519899) (end 101.1125 47.212399) (width 0.2) (layer "B.Cu") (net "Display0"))
 (segment (start 108.2375 22.088478) (end 108.2375 21.011522) (width 0.2) (layer "B.Cu") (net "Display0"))
 (segment (start 108.2375 21.011522) (end 111.469022 17.78) (width 0.2) (layer "B.Cu") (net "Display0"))
 (segment (start 126.107944 67.775) (end 118.277756 67.775) (width 0.2) (layer "B.Cu") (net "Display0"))
 (segment (start 144.375 24.515) (end 144.375 52.902056) (width 0.2) (layer "B.Cu") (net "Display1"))
 (segment (start 118.11207 68.175) (end 98.9125 48.97543) (width 0.2) (layer "B.Cu") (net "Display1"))
 (segment (start 100.6375 23.35) (end 105.2375 23.35) (width 0.2) (layer "B.Cu") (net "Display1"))
 (segment (start 136.098629 58.35) (end 126.273629 68.175) (width 0.2) (layer "B.Cu") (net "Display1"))
 (segment (start 144.375 52.902056) (end 138.927056 58.35) (width 0.2) (layer "B.Cu") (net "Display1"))
 (segment (start 113.3475 15.24) (end 115.85 15.24) (width 0.2) (layer "B.Cu") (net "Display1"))
 (segment (start 141.45 21.59) (end 144.375 24.515) (width 0.2) (layer "B.Cu") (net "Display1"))
 (segment (start 98.9125 48.97543) (end 98.9125 25.075) (width 0.2) (layer "B.Cu") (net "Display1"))
 (segment (start 126.273629 68.175) (end 118.11207 68.175) (width 0.2) (layer "B.Cu") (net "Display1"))
 (segment (start 98.9125 25.075) (end 100.6375 23.35) (width 0.2) (layer "B.Cu") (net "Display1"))
 (segment (start 138.927056 58.35) (end 136.098629 58.35) (width 0.2) (layer "B.Cu") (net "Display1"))
 (segment (start 105.2375 23.35) (end 113.3475 15.24) (width 0.2) (layer "B.Cu") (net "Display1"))
 (segment (start 124.1425 35.56) (end 123.825 35.2425) (width 0.2) (layer "F.Cu") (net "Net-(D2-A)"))
 (segment (start 129.54 35.56) (end 124.1425 35.56) (width 0.2) (layer "F.Cu") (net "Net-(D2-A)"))
 (segment (start 146.3675 33.3375) (end 142.875 33.3375) (width 0.2) (layer "F.Cu") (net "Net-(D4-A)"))
 (segment (start 148.59 35.56) (end 146.3675 33.3375) (width 0.2) (layer "F.Cu") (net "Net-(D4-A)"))
 (segment (start 156.0625 67.775) (end 139.2125 67.775) (width 0.2) (layer "F.Cu") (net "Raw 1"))
 (segment (start 139.2125 67.775) (end 138.1125 66.675) (width 0.2) (layer "F.Cu") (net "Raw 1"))
 (segment (start 157.1625 66.675) (end 156.0625 67.775) (width 0.2) (layer "F.Cu") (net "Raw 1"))
 (segment (start 119.0625 66.675) (end 111.89 59.5025) (width 0.2) (layer "F.Cu") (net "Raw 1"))
 (segment (start 138.1125 66.675) (end 137.0125 67.775) (width 0.2) (layer "F.Cu") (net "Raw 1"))
 (segment (start 120.1625 67.775) (end 119.0625 66.675) (width 0.2) (layer "F.Cu") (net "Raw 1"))
 (segment (start 111.89 59.5025) (end 111.89 49.957244) (width 0.2) (layer "F.Cu") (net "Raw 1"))
 (segment (start 111.89 49.957244) (end 100.0125 38.079744) (width 0.2) (layer "F.Cu") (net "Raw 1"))
 (segment (start 100.0125 38.079744) (end 100.0125 36.195) (width 0.2) (layer "F.Cu") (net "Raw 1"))
 (segment (start 137.0125 67.775) (end 120.1625 67.775) (width 0.2) (layer "F.Cu") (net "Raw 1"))
 (segment (start 141.45 26.67) (end 141.45 40.720101) (width 0.2) (layer "B.Cu") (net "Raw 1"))
 (segment (start 141.45 40.720101) (end 119.0625 63.107601) (width 0.2) (layer "B.Cu") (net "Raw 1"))
 (segment (start 119.0625 63.107601) (end 119.0625 66.675) (width 0.2) (layer "B.Cu") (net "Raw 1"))
 (segment (start 111.89 37.127056) (end 108.059556 40.9575) (width 0.2) (layer "F.Cu") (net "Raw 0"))
 (segment (start 154.360101 31.62) (end 150.05 35.930101) (width 0.2) (layer "F.Cu") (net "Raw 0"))
 (segment (start 146.159556 40.9575) (end 142.875 40.9575) (width 0.2) (layer "F.Cu") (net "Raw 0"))
 (segment (start 131 37.067056) (end 125.204556 42.8625) (width 0.2) (layer "F.Cu") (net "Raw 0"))
 (segment (start 136.469899 31.62) (end 135.310101 31.62) (width 0.2) (layer "F.Cu") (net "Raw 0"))
 (segment (start 123.825 38.025101) (end 117.419899 31.62) (width 0.2) (layer "F.Cu") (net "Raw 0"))
 (segment (start 150.05 37.067056) (end 146.159556 40.9575) (width 0.2) (layer "F.Cu") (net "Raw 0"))
 (segment (start 142.875 40.9575) (end 142.875 38.025101) (width 0.2) (layer "F.Cu") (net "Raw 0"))
 (segment (start 131 35.930101) (end 131 37.067056) (width 0.2) (layer "F.Cu") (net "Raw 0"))
 (segment (start 108.059556 40.9575) (end 104.775 40.9575) (width 0.2) (layer "F.Cu") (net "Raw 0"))
 (segment (start 125.204556 42.8625) (end 123.825 42.8625) (width 0.2) (layer "F.Cu") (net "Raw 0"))
 (segment (start 166.6875 36.195) (end 162.1125 31.62) (width 0.2) (layer "F.Cu") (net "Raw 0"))
 (segment (start 150.05 35.930101) (end 150.05 37.067056) (width 0.2) (layer "F.Cu") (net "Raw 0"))
 (segment (start 111.89 35.7475) (end 111.89 37.127056) (width 0.2) (layer "F.Cu") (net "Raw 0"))
 (segment (start 123.825 42.8625) (end 123.825 38.025101) (width 0.2) (layer "F.Cu") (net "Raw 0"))
 (segment (start 162.1125 31.62) (end 154.360101 31.62) (width 0.2) (layer "F.Cu") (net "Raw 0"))
 (segment (start 116.0175 31.62) (end 111.89 35.7475) (width 0.2) (layer "F.Cu") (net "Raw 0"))
 (segment (start 117.419899 31.62) (end 116.0175 31.62) (width 0.2) (layer "F.Cu") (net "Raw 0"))
 (segment (start 135.310101 31.62) (end 131 35.930101) (width 0.2) (layer "F.Cu") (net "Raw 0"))
 (segment (start 142.875 38.025101) (end 136.469899 31.62) (width 0.2) (layer "F.Cu") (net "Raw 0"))
 (segment (start 162.190686 7.425) (end 166.75 11.984315) (width 0.2) (layer "B.Cu") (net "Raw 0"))
 (segment (start 93.7375 15.25) (end 101.5625 7.425) (width 0.2) (layer "B.Cu") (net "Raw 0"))
 (segment (start 105.171814 22.85) (end 94.499022 22.85) (width 0.2) (layer "B.Cu") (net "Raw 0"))
 (segment (start 117 18.256346) (end 117 14.763654) (width 0.2) (layer "B.Cu") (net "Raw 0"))
 (segment (start 173.15 20.845837) (end 173.15 29.7325) (width 0.2) (layer "B.Cu") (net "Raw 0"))
 (segment (start 166.75 11.984315) (end 166.75 14.445837) (width 0.2) (layer "B.Cu") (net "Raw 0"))
 (segment (start 117 14.763654) (end 116.326346 14.09) (width 0.2) (layer "B.Cu") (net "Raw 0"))
 (segment (start 113.931814 14.09) (end 105.171814 22.85) (width 0.2) (layer "B.Cu") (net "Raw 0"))
 (segment (start 125.25 26.67) (end 117.064925 26.67) (width 0.2) (layer "B.Cu") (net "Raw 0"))
 (segment (start 110.884707 18.93) (end 116.326346 18.93) (width 0.2) (layer "B.Cu") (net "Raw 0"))
 (segment (start 110.104816 19.709891) (end 110.884707 18.93) (width 0.2) (layer "B.Cu") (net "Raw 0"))
 (segment (start 173.15 29.7325) (end 166.6875 36.195) (width 0.2) (layer "B.Cu") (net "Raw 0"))
 (segment (start 101.5625 7.425) (end 162.190686 7.425) (width 0.2) (layer "B.Cu") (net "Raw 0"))
 (segment (start 117.064925 26.67) (end 110.104816 19.709891) (width 0.2) (layer "B.Cu") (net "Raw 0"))
 (segment (start 94.499022 22.85) (end 93.7375 22.088478) (width 0.2) (layer "B.Cu") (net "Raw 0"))
 (segment (start 116.326346 18.93) (end 117 18.256346) (width 0.2) (layer "B.Cu") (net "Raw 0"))
 (segment (start 93.7375 22.088478) (end 93.7375 15.25) (width 0.2) (layer "B.Cu") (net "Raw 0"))
 (segment (start 166.75 14.445837) (end 173.15 20.845837) (width 0.2) (layer "B.Cu") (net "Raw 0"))
 (segment (start 116.326346 14.09) (end 113.931814 14.09) (width 0.2) (layer "B.Cu") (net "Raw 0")))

